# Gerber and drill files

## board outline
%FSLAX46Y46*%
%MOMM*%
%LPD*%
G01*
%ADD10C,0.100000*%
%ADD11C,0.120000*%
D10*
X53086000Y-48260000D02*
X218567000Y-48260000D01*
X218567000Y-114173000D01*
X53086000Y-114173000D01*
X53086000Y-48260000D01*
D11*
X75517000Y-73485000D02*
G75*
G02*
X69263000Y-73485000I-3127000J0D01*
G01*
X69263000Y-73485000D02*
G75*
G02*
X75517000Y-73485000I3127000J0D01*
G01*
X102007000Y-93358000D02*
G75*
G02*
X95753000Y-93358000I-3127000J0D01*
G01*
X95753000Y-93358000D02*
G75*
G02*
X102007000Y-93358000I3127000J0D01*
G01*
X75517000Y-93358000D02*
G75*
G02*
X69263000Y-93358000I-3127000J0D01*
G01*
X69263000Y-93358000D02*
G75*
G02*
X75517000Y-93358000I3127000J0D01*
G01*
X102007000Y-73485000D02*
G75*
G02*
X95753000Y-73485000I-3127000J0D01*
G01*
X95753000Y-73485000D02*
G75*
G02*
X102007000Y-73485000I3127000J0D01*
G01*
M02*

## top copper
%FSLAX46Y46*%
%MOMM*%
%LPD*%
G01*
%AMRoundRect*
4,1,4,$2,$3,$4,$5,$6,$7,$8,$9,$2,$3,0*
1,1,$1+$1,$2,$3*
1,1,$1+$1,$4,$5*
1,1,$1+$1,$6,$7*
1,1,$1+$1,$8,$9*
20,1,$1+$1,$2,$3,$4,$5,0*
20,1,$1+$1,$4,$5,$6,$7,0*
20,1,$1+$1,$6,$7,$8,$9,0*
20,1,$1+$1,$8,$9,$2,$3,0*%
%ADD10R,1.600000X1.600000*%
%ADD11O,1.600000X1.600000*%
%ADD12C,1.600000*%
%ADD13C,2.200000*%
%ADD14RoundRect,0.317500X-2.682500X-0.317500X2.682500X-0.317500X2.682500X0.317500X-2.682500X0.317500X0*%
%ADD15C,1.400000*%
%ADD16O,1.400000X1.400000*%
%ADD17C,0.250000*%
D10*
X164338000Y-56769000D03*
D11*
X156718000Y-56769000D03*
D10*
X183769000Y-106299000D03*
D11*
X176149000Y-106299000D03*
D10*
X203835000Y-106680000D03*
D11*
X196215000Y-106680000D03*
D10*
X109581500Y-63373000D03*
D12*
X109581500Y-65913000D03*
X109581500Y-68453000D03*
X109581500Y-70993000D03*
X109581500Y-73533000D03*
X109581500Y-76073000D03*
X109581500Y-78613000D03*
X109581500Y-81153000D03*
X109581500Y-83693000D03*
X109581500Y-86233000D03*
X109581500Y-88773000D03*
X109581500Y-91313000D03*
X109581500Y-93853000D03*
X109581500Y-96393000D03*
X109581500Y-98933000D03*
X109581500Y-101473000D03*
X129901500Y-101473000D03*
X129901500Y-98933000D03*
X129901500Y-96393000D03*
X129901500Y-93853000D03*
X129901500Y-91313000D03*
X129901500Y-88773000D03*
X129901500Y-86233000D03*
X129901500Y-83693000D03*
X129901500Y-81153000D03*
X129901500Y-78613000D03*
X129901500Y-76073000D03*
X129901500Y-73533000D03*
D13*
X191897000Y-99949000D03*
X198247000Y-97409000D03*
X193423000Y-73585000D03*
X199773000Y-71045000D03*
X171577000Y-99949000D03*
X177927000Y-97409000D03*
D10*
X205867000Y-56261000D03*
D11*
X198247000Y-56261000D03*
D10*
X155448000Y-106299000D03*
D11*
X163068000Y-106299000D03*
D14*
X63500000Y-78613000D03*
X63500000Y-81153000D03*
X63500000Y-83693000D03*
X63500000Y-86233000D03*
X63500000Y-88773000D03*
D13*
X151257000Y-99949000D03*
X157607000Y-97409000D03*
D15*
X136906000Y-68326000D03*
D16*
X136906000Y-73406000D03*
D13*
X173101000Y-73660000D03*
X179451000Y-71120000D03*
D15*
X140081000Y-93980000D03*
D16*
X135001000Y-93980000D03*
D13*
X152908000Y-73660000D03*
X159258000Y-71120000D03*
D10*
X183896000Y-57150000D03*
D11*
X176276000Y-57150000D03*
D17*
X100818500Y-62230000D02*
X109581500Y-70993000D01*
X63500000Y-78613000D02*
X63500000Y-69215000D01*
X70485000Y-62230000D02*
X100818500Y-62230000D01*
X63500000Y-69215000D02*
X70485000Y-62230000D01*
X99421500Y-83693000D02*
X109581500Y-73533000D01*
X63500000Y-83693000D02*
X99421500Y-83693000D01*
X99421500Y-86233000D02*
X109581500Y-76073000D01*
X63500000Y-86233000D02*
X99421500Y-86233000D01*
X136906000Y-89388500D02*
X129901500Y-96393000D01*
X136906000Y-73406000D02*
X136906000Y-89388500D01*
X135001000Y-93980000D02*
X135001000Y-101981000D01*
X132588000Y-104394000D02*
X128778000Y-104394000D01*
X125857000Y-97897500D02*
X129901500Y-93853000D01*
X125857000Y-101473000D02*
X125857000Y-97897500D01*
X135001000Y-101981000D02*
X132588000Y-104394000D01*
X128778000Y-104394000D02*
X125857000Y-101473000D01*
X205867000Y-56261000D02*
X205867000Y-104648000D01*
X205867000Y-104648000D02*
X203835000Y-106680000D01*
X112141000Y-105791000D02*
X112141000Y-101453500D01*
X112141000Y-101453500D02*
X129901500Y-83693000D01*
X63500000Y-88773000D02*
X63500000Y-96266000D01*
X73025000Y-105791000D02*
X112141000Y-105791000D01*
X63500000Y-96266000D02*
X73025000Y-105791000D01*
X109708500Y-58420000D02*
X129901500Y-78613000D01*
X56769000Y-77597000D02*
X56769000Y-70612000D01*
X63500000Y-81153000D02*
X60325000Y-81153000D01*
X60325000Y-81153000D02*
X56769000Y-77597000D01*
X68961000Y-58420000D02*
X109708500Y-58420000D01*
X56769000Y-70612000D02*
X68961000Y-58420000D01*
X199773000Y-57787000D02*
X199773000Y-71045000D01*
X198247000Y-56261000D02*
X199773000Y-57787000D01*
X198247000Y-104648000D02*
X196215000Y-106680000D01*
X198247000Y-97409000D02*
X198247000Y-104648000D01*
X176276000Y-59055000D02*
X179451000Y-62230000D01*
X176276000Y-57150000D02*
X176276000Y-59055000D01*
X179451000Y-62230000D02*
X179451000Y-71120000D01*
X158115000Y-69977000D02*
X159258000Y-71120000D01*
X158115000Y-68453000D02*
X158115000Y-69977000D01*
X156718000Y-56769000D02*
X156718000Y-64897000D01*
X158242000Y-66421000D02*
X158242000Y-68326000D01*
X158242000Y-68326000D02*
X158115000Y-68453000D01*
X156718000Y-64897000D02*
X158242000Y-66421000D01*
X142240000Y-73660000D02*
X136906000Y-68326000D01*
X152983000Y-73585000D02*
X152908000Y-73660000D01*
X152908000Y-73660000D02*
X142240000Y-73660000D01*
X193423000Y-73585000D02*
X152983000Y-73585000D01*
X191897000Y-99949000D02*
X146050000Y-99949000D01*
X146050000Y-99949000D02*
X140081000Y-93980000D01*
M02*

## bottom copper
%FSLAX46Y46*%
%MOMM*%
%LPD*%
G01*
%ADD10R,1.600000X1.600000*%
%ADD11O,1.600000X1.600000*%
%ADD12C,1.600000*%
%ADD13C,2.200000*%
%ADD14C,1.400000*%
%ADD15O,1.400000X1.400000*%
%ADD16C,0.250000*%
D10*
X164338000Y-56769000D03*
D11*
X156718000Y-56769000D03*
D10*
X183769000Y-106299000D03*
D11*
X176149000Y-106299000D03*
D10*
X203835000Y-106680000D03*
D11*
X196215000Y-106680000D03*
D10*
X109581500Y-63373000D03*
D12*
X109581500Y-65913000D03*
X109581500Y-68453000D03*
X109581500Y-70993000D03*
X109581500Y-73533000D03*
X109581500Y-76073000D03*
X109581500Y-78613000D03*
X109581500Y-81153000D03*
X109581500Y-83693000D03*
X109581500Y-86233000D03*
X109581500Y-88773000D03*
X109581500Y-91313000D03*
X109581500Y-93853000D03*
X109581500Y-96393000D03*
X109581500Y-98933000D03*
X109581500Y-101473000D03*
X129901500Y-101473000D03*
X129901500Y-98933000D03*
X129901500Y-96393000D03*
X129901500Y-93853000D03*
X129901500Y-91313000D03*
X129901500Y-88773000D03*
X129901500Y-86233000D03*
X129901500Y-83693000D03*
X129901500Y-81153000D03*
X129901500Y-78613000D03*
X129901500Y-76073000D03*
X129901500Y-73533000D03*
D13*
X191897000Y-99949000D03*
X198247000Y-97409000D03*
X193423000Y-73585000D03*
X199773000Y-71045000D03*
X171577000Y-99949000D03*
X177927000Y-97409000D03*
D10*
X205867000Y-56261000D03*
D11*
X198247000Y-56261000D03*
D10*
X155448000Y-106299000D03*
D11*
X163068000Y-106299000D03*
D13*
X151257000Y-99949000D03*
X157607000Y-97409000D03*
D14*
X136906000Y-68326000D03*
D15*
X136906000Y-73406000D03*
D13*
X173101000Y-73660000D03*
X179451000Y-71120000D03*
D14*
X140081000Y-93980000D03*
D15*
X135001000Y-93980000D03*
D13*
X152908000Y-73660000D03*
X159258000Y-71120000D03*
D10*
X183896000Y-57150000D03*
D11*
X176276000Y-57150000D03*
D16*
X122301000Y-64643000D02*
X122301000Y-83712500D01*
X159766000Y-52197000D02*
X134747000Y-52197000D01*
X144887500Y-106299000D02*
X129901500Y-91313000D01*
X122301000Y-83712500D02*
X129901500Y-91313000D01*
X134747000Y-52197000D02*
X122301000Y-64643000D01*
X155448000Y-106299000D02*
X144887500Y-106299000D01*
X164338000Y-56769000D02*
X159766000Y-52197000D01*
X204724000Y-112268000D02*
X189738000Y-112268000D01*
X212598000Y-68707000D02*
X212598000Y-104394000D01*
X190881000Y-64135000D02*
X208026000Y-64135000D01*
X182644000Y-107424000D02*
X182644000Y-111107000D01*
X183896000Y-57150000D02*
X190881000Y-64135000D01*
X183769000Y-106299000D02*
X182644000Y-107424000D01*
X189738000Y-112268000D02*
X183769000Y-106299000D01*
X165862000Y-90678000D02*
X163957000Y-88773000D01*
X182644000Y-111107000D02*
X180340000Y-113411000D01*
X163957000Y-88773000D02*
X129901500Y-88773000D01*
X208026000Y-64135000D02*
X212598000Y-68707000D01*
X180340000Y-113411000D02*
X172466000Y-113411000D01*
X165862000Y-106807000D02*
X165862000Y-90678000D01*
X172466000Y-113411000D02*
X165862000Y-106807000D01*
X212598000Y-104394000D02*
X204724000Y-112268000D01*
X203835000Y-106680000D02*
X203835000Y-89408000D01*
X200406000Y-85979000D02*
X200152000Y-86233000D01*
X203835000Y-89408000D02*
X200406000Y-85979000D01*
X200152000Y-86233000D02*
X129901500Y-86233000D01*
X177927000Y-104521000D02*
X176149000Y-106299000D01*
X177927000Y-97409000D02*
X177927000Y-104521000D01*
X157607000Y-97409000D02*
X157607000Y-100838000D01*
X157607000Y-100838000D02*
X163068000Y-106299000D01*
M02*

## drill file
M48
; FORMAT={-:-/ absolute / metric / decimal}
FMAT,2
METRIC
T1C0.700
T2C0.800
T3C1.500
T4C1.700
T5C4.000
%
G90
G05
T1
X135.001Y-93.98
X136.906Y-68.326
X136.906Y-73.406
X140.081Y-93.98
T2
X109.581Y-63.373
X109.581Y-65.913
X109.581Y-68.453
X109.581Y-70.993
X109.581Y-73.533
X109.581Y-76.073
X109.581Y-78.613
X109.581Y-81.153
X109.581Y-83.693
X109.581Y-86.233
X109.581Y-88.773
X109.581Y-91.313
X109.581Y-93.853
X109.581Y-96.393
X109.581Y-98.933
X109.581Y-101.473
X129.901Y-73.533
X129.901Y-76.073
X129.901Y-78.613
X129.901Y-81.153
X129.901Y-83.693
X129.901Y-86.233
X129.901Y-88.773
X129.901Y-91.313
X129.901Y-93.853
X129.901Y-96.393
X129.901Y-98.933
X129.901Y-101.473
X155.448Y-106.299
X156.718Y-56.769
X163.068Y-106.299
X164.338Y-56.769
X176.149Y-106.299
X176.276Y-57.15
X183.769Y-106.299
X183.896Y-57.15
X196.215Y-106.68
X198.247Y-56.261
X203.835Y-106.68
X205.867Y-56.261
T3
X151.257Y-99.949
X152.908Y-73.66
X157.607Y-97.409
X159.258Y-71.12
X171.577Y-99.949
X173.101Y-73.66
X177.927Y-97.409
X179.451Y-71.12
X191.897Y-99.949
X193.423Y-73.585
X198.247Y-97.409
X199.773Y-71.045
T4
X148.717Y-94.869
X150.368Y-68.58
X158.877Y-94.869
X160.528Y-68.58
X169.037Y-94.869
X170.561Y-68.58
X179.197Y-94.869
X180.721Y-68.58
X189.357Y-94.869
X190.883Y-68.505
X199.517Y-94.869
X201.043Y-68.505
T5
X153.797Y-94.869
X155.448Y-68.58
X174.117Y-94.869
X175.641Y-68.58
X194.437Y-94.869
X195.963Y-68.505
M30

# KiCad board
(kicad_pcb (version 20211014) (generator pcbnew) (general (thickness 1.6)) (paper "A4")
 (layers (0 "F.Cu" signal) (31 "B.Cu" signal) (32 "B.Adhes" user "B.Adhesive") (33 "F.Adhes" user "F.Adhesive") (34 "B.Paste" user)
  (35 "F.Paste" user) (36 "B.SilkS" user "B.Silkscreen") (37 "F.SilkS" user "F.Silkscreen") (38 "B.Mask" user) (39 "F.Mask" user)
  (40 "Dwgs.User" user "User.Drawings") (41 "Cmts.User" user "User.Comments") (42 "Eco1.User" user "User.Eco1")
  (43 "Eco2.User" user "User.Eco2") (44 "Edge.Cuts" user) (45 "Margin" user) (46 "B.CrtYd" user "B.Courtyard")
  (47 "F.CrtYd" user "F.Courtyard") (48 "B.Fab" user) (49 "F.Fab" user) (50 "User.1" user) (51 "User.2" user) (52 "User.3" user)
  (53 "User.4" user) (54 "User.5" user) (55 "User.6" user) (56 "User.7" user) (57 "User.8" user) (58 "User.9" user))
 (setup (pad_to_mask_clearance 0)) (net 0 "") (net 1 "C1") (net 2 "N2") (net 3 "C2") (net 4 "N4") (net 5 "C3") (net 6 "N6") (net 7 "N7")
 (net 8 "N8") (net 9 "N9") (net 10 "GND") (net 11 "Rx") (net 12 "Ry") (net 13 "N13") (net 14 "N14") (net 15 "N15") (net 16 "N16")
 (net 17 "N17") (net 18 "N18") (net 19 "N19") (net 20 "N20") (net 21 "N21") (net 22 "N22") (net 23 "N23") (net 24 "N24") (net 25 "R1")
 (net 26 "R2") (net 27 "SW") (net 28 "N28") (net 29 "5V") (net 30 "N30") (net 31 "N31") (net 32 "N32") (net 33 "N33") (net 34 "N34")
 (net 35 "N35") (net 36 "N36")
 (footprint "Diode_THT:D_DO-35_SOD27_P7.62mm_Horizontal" (layer "F.Cu") (at 164.338 56.769 180)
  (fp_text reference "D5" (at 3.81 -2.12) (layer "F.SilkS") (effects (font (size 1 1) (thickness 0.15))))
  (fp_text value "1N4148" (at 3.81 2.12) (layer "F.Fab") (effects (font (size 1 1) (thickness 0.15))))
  (pad "1" thru_hole rect (at 0 0 180) (size 1.6 1.6) (drill 0.8) (layers *.Cu *.Mask) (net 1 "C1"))
  (pad "2" thru_hole oval (at 7.62 0 180) (size 1.6 1.6) (drill 0.8) (layers *.Cu *.Mask) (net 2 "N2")))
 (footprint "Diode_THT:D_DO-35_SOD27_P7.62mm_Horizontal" (layer "F.Cu") (at 183.769 106.299 180)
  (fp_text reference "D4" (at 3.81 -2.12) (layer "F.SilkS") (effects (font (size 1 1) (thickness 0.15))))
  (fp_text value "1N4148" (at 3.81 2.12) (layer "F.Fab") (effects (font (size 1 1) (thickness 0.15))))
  (pad "1" thru_hole rect (at 0 0 180) (size 1.6 1.6) (drill 0.8) (layers *.Cu *.Mask) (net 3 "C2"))
  (pad "2" thru_hole oval (at 7.62 0 180) (size 1.6 1.6) (drill 0.8) (layers *.Cu *.Mask) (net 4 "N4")))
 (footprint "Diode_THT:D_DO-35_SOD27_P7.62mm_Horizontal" (layer "F.Cu") (at 203.835 106.68 180)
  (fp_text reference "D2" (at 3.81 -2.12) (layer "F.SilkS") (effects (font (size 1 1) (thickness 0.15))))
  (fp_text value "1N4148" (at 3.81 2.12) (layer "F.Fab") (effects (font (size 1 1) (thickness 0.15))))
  (pad "1" thru_hole rect (at 0 0 180) (size 1.6 1.6) (drill 0.8) (layers *.Cu *.Mask) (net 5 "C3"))
  (pad "2" thru_hole oval (at 7.62 0 180) (size 1.6 1.6) (drill 0.8) (layers *.Cu *.Mask) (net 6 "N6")))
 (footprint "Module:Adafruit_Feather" (layer "F.Cu") (at 109.5815 63.373)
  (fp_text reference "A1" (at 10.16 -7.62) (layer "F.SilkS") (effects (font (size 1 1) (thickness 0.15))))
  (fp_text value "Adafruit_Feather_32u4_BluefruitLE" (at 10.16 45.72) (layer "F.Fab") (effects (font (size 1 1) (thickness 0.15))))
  (pad "1" thru_hole rect (at 0 0 180) (size 1.6 1.6) (drill 0.8) (layers *.Cu *.Mask) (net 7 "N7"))
  (pad "2" thru_hole circle (at 0 2.54 180) (size 1.6 1.6) (drill 0.8) (layers *.Cu *.Mask) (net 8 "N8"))
  (pad "3" thru_hole circle (at 0 5.08 180) (size 1.6 1.6) (drill 0.8) (layers *.Cu *.Mask) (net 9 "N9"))
  (pad "4" thru_hole circle (at 0 7.62 180) (size 1.6 1.6) (drill 0.8) (layers *.Cu *.Mask) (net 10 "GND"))
  (pad "5" thru_hole circle (at 0 10.16 180) (size 1.6 1.6) (drill 0.8) (layers *.Cu *.Mask) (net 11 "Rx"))
  (pad "6" thru_hole circle (at 0 12.7 180) (size 1.6 1.6) (drill 0.8) (layers *.Cu *.Mask) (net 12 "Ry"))
  (pad "7" thru_hole circle (at 0 15.24 180) (size 1.6 1.6) (drill 0.8) (layers *.Cu *.Mask) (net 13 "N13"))
  (pad "8" thru_hole circle (at 0 17.78 180) (size 1.6 1.6) (drill 0.8) (layers *.Cu *.Mask) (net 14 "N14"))
  (pad "9" thru_hole circle (at 0 20.32 180) (size 1.6 1.6) (drill 0.8) (layers *.Cu *.Mask) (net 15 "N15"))
  (pad "10" thru_hole circle (at 0 22.86 180) (size 1.6 1.6) (drill 0.8) (layers *.Cu *.Mask) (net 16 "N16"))
  (pad "11" thru_hole circle (at 0 25.4 180) (size 1.6 1.6) (drill 0.8) (layers *.Cu *.Mask) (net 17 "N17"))
  (pad "12" thru_hole circle (at 0 27.94 180) (size 1.6 1.6) (drill 0.8) (layers *.Cu *.Mask) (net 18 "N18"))
  (pad "13" thru_hole circle (at 0 30.48 180) (size 1.6 1.6) (drill 0.8) (layers *.Cu *.Mask) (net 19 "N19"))
  (pad "14" thru_hole circle (at 0 33.02 180) (size 1.6 1.6) (drill 0.8) (layers *.Cu *.Mask) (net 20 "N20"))
  (pad "15" thru_hole circle (at 0 35.56 180) (size 1.6 1.6) (drill 0.8) (layers *.Cu *.Mask) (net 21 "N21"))
  (pad "16" thru_hole circle (at 0 38.1 180) (size 1.6 1.6) (drill 0.8) (layers *.Cu *.Mask) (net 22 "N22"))
  (pad "17" thru_hole circle (at 20.32 38.1 180) (size 1.6 1.6) (drill 0.8) (layers *.Cu *.Mask) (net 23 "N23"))
  (pad "18" thru_hole circle (at 20.32 35.56 180) (size 1.6 1.6) (drill 0.8) (layers *.Cu *.Mask) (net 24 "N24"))
  (pad "19" thru_hole circle (at 20.32 33.02 180) (size 1.6 1.6) (drill 0.8) (layers *.Cu *.Mask) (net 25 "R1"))
  (pad "20" thru_hole circle (at 20.32 30.48 180) (size 1.6 1.6) (drill 0.8) (layers *.Cu *.Mask) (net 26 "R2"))
  (pad "21" thru_hole circle (at 20.32 27.94 180) (size 1.6 1.6) (drill 0.8) (layers *.Cu *.Mask) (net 1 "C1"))
  (pad "22" thru_hole circle (at 20.32 25.4 180) (size 1.6 1.6) (drill 0.8) (layers *.Cu *.Mask) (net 3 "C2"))
  (pad "23" thru_hole circle (at 20.32 22.86 180) (size 1.6 1.6) (drill 0.8) (layers *.Cu *.Mask) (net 5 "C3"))
  (pad "24" thru_hole circle (at 20.32 20.32 180) (size 1.6 1.6) (drill 0.8) (layers *.Cu *.Mask) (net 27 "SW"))
  (pad "25" thru_hole circle (at 20.32 17.78 180) (size 1.6 1.6) (drill 0.8) (layers *.Cu *.Mask) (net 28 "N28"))
  (pad "26" thru_hole circle (at 20.32 15.24 180) (size 1.6 1.6) (drill 0.8) (layers *.Cu *.Mask) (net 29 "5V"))
  (pad "27" thru_hole circle (at 20.32 12.7 180) (size 1.6 1.6) (drill 0.8) (layers *.Cu *.Mask) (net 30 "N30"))
  (pad "28" thru_hole circle (at 20.32 10.16 180) (size 1.6 1.6) (drill 0.8) (layers *.Cu *.Mask) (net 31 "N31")))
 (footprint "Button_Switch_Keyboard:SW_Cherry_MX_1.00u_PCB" (layer "F.Cu") (at 191.897 99.949 180)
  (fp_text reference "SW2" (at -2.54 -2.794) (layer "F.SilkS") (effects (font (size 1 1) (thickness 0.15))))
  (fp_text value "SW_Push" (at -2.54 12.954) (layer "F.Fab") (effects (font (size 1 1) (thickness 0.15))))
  (pad "" np_thru_hole circle (at 2.54 5.08 180) (size 1.7 1.7) (drill 1.7) (layers *.Cu *.Mask))
  (pad "" np_thru_hole circle (at -2.54 5.08 180) (size 4 4) (drill 4) (layers *.Cu *.Mask))
  (pad "" np_thru_hole circle (at -7.62 5.08 180) (size 1.7 1.7) (drill 1.7) (layers *.Cu *.Mask))
  (pad "1" thru_hole circle (at 0 0 180) (size 2.2 2.2) (drill 1.5) (layers *.Cu *.Mask) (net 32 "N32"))
  (pad "2" thru_hole circle (at -6.35 2.54 180) (size 2.2 2.2) (drill 1.5) (layers *.Cu *.Mask) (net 6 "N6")))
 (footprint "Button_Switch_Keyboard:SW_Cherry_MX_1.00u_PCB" (layer "F.Cu") (at 193.423 73.585 180)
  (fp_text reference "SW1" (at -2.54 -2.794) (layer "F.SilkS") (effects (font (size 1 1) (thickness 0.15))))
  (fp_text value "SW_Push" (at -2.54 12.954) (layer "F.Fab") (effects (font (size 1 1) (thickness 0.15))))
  (pad "" np_thru_hole circle (at -2.54 5.08 180) (size 4 4) (drill 4) (layers *.Cu *.Mask))
  (pad "" np_thru_hole circle (at -7.62 5.08 180) (size 1.7 1.7) (drill 1.7) (layers *.Cu *.Mask))
  (pad "" np_thru_hole circle (at 2.54 5.08 180) (size 1.7 1.7) (drill 1.7) (layers *.Cu *.Mask))
  (pad "1" thru_hole circle (at 0 0 180) (size 2.2 2.2) (drill 1.5) (layers *.Cu *.Mask) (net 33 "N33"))
  (pad "2" thru_hole circle (at -6.35 2.54 180) (size 2.2 2.2) (drill 1.5) (layers *.Cu *.Mask) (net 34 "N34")))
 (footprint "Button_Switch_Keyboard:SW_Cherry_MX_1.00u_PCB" (layer "F.Cu") (at 171.577 99.949 180)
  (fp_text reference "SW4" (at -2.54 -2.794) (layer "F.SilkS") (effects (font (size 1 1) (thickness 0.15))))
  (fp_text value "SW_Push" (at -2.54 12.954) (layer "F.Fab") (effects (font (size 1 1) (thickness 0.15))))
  (pad "" np_thru_hole circle (at -7.62 5.08 180) (size 1.7 1.7) (drill 1.7) (layers *.Cu *.Mask))
  (pad "" np_thru_hole circle (at 2.54 5.08 180) (size 1.7 1.7) (drill 1.7) (layers *.Cu *.Mask))
  (pad "" np_thru_hole circle (at -2.54 5.08 180) (size 4 4) (drill 4) (layers *.Cu *.Mask))
  (pad "1" thru_hole circle (at 0 0 180) (size 2.2 2.2) (drill 1.5) (layers *.Cu *.Mask) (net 32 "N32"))
  (pad "2" thru_hole circle (at -6.35 2.54 180) (size 2.2 2.2) (drill 1.5) (layers *.Cu *.Mask) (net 4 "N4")))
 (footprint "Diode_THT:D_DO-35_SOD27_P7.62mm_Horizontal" (layer "F.Cu") (at 205.867 56.261 180)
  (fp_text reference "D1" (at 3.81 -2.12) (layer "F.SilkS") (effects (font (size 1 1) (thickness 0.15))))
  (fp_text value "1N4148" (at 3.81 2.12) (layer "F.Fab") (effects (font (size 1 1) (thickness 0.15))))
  (pad "1" thru_hole rect (at 0 0 180) (size 1.6 1.6) (drill 0.8) (layers *.Cu *.Mask) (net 5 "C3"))
  (pad "2" thru_hole oval (at 7.62 0 180) (size 1.6 1.6) (drill 0.8) (layers *.Cu *.Mask) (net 34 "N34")))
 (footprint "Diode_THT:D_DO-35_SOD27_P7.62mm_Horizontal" (layer "F.Cu") (at 155.448 106.299)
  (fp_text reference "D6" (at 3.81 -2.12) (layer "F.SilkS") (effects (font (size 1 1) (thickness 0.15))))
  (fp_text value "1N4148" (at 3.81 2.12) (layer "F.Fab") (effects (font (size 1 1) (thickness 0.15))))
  (pad "1" thru_hole rect (at 0 0) (size 1.6 1.6) (drill 0.8) (layers *.Cu *.Mask) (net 1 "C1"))
  (pad "2" thru_hole oval (at 7.62 0) (size 1.6 1.6) (drill 0.8) (layers *.Cu *.Mask) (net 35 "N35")))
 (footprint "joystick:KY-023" (layer "F.Cu") (at 68.58 70.358)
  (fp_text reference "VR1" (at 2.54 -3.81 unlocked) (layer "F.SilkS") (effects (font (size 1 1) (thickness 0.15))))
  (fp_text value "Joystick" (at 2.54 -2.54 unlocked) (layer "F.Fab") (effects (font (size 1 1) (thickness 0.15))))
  (fp_circle (center 3.81 3.127) (end 6.937 3.127) (layer "Edge.Cuts") (width 0.12) (fill none))
  (fp_circle (center 30.3 23) (end 33.427 23) (layer "Edge.Cuts") (width 0.12) (fill none))
  (fp_circle (center 3.81 23) (end 6.937 23) (layer "Edge.Cuts") (width 0.12) (fill none))
  (fp_circle (center 30.3 3.127) (end 33.427 3.127) (layer "Edge.Cuts") (width 0.12) (fill none))
  (pad "1" smd roundrect (at -5.08 8.255) (size 6 1.27) (layers "F.Cu" "F.Paste" "F.Mask") (roundrect_rratio 0.25) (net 10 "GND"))
  (pad "2" smd roundrect (at -5.08 10.795) (size 6 1.27) (layers "F.Cu" "F.Paste" "F.Mask") (roundrect_rratio 0.25) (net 29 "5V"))
  (pad "3" smd roundrect (at -5.08 13.335) (size 6 1.27) (layers "F.Cu" "F.Paste" "F.Mask") (roundrect_rratio 0.25) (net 11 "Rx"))
  (pad "4" smd roundrect (at -5.08 15.875) (size 6 1.27) (layers "F.Cu" "F.Paste" "F.Mask") (roundrect_rratio 0.25) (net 12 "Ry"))
  (pad "5" smd roundrect (at -5.08 18.415) (size 6 1.27) (layers "F.Cu" "F.Paste" "F.Mask") (roundrect_rratio 0.25) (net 27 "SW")))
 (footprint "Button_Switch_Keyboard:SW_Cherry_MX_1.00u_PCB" (layer "F.Cu") (at 151.257 99.949 180)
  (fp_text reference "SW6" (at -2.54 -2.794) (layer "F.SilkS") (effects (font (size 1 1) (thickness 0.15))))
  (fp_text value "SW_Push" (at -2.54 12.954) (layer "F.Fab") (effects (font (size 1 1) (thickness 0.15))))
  (pad "" np_thru_hole circle (at 2.54 5.08 180) (size 1.7 1.7) (drill 1.7) (layers *.Cu *.Mask))
  (pad "" np_thru_hole circle (at -7.62 5.08 180) (size 1.7 1.7) (drill 1.7) (layers *.Cu *.Mask))
  (pad "" np_thru_hole circle (at -2.54 5.08 180) (size 4 4) (drill 4) (layers *.Cu *.Mask))
  (pad "1" thru_hole circle (at 0 0 180) (size 2.2 2.2) (drill 1.5) (layers *.Cu *.Mask) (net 32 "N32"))
  (pad "2" thru_hole circle (at -6.35 2.54 180) (size 2.2 2.2) (drill 1.5) (layers *.Cu *.Mask) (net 35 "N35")))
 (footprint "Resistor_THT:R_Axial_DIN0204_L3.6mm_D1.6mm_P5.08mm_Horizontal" (layer "F.Cu") (at 136.906 68.326 -90)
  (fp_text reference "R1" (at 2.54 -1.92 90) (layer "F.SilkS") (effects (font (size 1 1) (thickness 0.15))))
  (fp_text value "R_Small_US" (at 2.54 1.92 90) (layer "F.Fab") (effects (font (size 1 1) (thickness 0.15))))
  (pad "1" thru_hole circle (at 0 0 270) (size 1.4 1.4) (drill 0.7) (layers *.Cu *.Mask) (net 33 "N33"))
  (pad "2" thru_hole oval (at 5.08 0 270) (size 1.4 1.4) (drill 0.7) (layers *.Cu *.Mask) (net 25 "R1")))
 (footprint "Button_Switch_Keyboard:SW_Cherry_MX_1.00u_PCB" (layer "F.Cu") (at 173.101 73.66 180)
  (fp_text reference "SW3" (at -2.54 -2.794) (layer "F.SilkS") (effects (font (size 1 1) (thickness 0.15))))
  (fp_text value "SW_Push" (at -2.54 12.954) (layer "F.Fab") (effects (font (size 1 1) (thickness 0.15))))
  (pad "" np_thru_hole circle (at 2.54 5.08 180) (size 1.7 1.7) (drill 1.7) (layers *.Cu *.Mask))
  (pad "" np_thru_hole circle (at -2.54 5.08 180) (size 4 4) (drill 4) (layers *.Cu *.Mask))
  (pad "" np_thru_hole circle (at -7.62 5.08 180) (size 1.7 1.7) (drill 1.7) (layers *.Cu *.Mask))
  (pad "1" thru_hole circle (at 0 0 180) (size 2.2 2.2) (drill 1.5) (layers *.Cu *.Mask) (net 33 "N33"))
  (pad "2" thru_hole circle (at -6.35 2.54 180) (size 2.2 2.2) (drill 1.5) (layers *.Cu *.Mask) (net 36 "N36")))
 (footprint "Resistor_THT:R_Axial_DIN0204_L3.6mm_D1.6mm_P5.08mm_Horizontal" (layer "F.Cu") (at 140.081 93.98 180)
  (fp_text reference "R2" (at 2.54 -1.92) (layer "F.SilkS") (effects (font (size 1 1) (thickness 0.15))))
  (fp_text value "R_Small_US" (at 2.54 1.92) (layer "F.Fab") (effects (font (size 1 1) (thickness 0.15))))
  (pad "1" thru_hole circle (at 0 0 180) (size 1.4 1.4) (drill 0.7) (layers *.Cu *.Mask) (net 32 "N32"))
  (pad "2" thru_hole oval (at 5.08 0 180) (size 1.4 1.4) (drill 0.7) (layers *.Cu *.Mask) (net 26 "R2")))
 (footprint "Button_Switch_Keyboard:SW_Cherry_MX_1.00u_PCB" (layer "F.Cu") (at 152.908 73.66 180)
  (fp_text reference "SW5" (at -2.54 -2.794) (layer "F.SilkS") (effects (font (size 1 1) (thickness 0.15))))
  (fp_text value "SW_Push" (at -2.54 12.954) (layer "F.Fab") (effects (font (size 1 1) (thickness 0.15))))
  (pad "" np_thru_hole circle (at 2.54 5.08 180) (size 1.7 1.7) (drill 1.7) (layers *.Cu *.Mask))
  (pad "" np_thru_hole circle (at -2.54 5.08 180) (size 4 4) (drill 4) (layers *.Cu *.Mask))
  (pad "" np_thru_hole circle (at -7.62 5.08 180) (size 1.7 1.7) (drill 1.7) (layers *.Cu *.Mask))
  (pad "1" thru_hole circle (at 0 0 180) (size 2.2 2.2) (drill 1.5) (layers *.Cu *.Mask) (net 33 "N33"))
  (pad "2" thru_hole circle (at -6.35 2.54 180) (size 2.2 2.2) (drill 1.5) (layers *.Cu *.Mask) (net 2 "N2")))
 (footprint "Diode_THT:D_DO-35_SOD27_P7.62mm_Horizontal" (layer "F.Cu") (at 183.896 57.15 180)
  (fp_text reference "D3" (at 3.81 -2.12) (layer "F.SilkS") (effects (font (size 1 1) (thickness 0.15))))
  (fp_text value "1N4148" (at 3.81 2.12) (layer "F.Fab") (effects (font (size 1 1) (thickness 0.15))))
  (pad "1" thru_hole rect (at 0 0 180) (size 1.6 1.6) (drill 0.8) (layers *.Cu *.Mask) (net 3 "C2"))
  (pad "2" thru_hole oval (at 7.62 0 180) (size 1.6 1.6) (drill 0.8) (layers *.Cu *.Mask) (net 36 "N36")))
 (gr_rect (start 218.567 114.173) (end 53.086 48.26) (layer "Edge.Cuts") (width 0.1) (fill none))
 (segment (start 100.8185 62.23) (end 109.5815 70.993) (width 0.25) (layer "F.Cu") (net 10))
 (segment (start 63.5 78.613) (end 63.5 69.215) (width 0.25) (layer "F.Cu") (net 10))
 (segment (start 70.485 62.23) (end 100.8185 62.23) (width 0.25) (layer "F.Cu") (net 10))
 (segment (start 63.5 69.215) (end 70.485 62.23) (width 0.25) (layer "F.Cu") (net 10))
 (segment (start 99.4215 83.693) (end 109.5815 73.533) (width 0.25) (layer "F.Cu") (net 11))
 (segment (start 63.5 83.693) (end 99.4215 83.693) (width 0.25) (layer "F.Cu") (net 11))
 (segment (start 99.4215 86.233) (end 109.5815 76.073) (width 0.25) (layer "F.Cu") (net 12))
 (segment (start 63.5 86.233) (end 99.4215 86.233) (width 0.25) (layer "F.Cu") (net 12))
 (segment (start 136.906 89.3885) (end 129.9015 96.393) (width 0.25) (layer "F.Cu") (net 25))
 (segment (start 136.906 73.406) (end 136.906 89.3885) (width 0.25) (layer "F.Cu") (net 25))
 (segment (start 135.001 93.98) (end 135.001 101.981) (width 0.25) (layer "F.Cu") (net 26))
 (segment (start 132.588 104.394) (end 128.778 104.394) (width 0.25) (layer "F.Cu") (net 26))
 (segment (start 125.857 97.8975) (end 129.9015 93.853) (width 0.25) (layer "F.Cu") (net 26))
 (segment (start 125.857 101.473) (end 125.857 97.8975) (width 0.25) (layer "F.Cu") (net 26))
 (segment (start 135.001 101.981) (end 132.588 104.394) (width 0.25) (layer "F.Cu") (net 26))
 (segment (start 128.778 104.394) (end 125.857 101.473) (width 0.25) (layer "F.Cu") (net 26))
 (segment (start 122.301 64.643) (end 122.301 83.7125) (width 0.25) (layer "B.Cu") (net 1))
 (segment (start 159.766 52.197) (end 134.747 52.197) (width 0.25) (layer "B.Cu") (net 1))
 (segment (start 144.8875 106.299) (end 129.9015 91.313) (width 0.25) (layer "B.Cu") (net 1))
 (segment (start 122.301 83.7125) (end 129.9015 91.313) (width 0.25) (layer "B.Cu") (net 1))
 (segment (start 134.747 52.197) (end 122.301 64.643) (width 0.25) (layer "B.Cu") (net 1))
 (segment (start 155.448 106.299) (end 144.8875 106.299) (width 0.25) (layer "B.Cu") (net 1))
 (segment (start 164.338 56.769) (end 159.766 52.197) (width 0.25) (layer "B.Cu") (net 1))
 (segment (start 204.724 112.268) (end 189.738 112.268) (width 0.25) (layer "B.Cu") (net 3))
 (segment (start 212.598 68.707) (end 212.598 104.394) (width 0.25) (layer "B.Cu") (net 3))
 (segment (start 190.881 64.135) (end 208.026 64.135) (width 0.25) (layer "B.Cu") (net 3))
 (segment (start 182.644 107.424) (end 182.644 111.107) (width 0.25) (layer "B.Cu") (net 3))
 (segment (start 183.896 57.15) (end 190.881 64.135) (width 0.25) (layer "B.Cu") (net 3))
 (segment (start 183.769 106.299) (end 182.644 107.424) (width 0.25) (layer "B.Cu") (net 3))
 (segment (start 189.738 112.268) (end 183.769 106.299) (width 0.25) (layer "B.Cu") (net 3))
 (segment (start 165.862 90.678) (end 163.957 88.773) (width 0.25) (layer "B.Cu") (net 3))
 (segment (start 182.644 111.107) (end 180.34 113.411) (width 0.25) (layer "B.Cu") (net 3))
 (segment (start 163.957 88.773) (end 129.9015 88.773) (width 0.25) (layer "B.Cu") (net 3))
 (segment (start 208.026 64.135) (end 212.598 68.707) (width 0.25) (layer "B.Cu") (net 3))
 (segment (start 180.34 113.411) (end 172.466 113.411) (width 0.25) (layer "B.Cu") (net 3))
 (segment (start 165.862 106.807) (end 165.862 90.678) (width 0.25) (layer "B.Cu") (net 3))
 (segment (start 172.466 113.411) (end 165.862 106.807) (width 0.25) (layer "B.Cu") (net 3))
 (segment (start 212.598 104.394) (end 204.724 112.268) (width 0.25) (layer "B.Cu") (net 3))
 (segment (start 205.867 56.261) (end 205.867 104.648) (width 0.25) (layer "F.Cu") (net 5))
 (segment (start 205.867 104.648) (end 203.835 106.68) (width 0.25) (layer "F.Cu") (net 5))
 (segment (start 203.835 106.68) (end 203.835 89.408) (width 0.25) (layer "B.Cu") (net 5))
 (segment (start 200.406 85.979) (end 200.152 86.233) (width 0.25) (layer "B.Cu") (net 5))
 (segment (start 203.835 89.408) (end 200.406 85.979) (width 0.25) (layer "B.Cu") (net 5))
 (segment (start 200.152 86.233) (end 129.9015 86.233) (width 0.25) (layer "B.Cu") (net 5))
 (segment (start 112.141 105.791) (end 112.141 101.4535) (width 0.25) (layer "F.Cu") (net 27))
 (segment (start 112.141 101.4535) (end 129.9015 83.693) (width 0.25) (layer "F.Cu") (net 27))
 (segment (start 63.5 88.773) (end 63.5 96.266) (width 0.25) (layer "F.Cu") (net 27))
 (segment (start 73.025 105.791) (end 112.141 105.791) (width 0.25) (layer "F.Cu") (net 27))
 (segment (start 63.5 96.266) (end 73.025 105.791) (width 0.25) (layer "F.Cu") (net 27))
 (segment (start 109.7085 58.42) (end 129.9015 78.613) (width 0.25) (layer "F.Cu") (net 29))
 (segment (start 56.769 77.597) (end 56.769 70.612) (width 0.25) (layer "F.Cu") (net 29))
 (segment (start 63.5 81.153) (end 60.325 81.153) (width 0.25) (layer "F.Cu") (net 29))
 (segment (start 60.325 81.153) (end 56.769 77.597) (width 0.25) (layer "F.Cu") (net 29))
 (segment (start 68.961 58.42) (end 109.7085 58.42) (width 0.25) (layer "F.Cu") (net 29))
 (segment (start 56.769 70.612) (end 68.961 58.42) (width 0.25) (layer "F.Cu") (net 29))
 (segment (start 199.773 57.787) (end 199.773 71.045) (width 0.25) (layer "F.Cu") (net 34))
 (segment (start 198.247 56.261) (end 199.773 57.787) (width 0.25) (layer "F.Cu") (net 34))
 (segment (start 198.247 104.648) (end 196.215 106.68) (width 0.25) (layer "F.Cu") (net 6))
 (segment (start 198.247 97.409) (end 198.247 104.648) (width 0.25) (layer "F.Cu") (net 6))
 (segment (start 176.276 59.055) (end 179.451 62.23) (width 0.25) (layer "F.Cu") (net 36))
 (segment (start 176.276 57.15) (end 176.276 59.055) (width 0.25) (layer "F.Cu") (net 36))
 (segment (start 179.451 62.23) (end 179.451 71.12) (width 0.25) (layer "F.Cu") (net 36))
 (segment (start 177.927 104.521) (end 176.149 106.299) (width 0.25) (layer "B.Cu") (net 4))
 (segment (start 177.927 97.409) (end 177.927 104.521) (width 0.25) (layer "B.Cu") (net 4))
 (segment (start 158.115 69.977) (end 159.258 71.12) (width 0.25) (layer "F.Cu") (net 2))
 (segment (start 158.115 68.453) (end 158.115 69.977) (width 0.25) (layer "F.Cu") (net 2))
 (segment (start 156.718 56.769) (end 156.718 64.897) (width 0.25) (layer "F.Cu") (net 2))
 (segment (start 158.242 66.421) (end 158.242 68.326) (width 0.25) (layer "F.Cu") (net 2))
 (segment (start 158.242 68.326) (end 158.115 68.453) (width 0.25) (layer "F.Cu") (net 2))
 (segment (start 156.718 64.897) (end 158.242 66.421) (width 0.25) (layer "F.Cu") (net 2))
 (segment (start 157.607 97.409) (end 157.607 100.838) (width 0.25) (layer "B.Cu") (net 35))
 (segment (start 157.607 100.838) (end 163.068 106.299) (width 0.25) (layer "B.Cu") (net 35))
 (segment (start 142.24 73.66) (end 136.906 68.326) (width 0.25) (layer "F.Cu") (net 33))
 (segment (start 152.983 73.585) (end 152.908 73.66) (width 0.25) (layer "F.Cu") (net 33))
 (segment (start 152.908 73.66) (end 142.24 73.66) (width 0.25) (layer "F.Cu") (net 33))
 (segment (start 193.423 73.585) (end 152.983 73.585) (width 0.25) (layer "F.Cu") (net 33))
 (segment (start 191.897 99.949) (end 146.05 99.949) (width 0.25) (layer "F.Cu") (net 32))
 (segment (start 146.05 99.949) (end 140.081 93.98) (width 0.25) (layer "F.Cu") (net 32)))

